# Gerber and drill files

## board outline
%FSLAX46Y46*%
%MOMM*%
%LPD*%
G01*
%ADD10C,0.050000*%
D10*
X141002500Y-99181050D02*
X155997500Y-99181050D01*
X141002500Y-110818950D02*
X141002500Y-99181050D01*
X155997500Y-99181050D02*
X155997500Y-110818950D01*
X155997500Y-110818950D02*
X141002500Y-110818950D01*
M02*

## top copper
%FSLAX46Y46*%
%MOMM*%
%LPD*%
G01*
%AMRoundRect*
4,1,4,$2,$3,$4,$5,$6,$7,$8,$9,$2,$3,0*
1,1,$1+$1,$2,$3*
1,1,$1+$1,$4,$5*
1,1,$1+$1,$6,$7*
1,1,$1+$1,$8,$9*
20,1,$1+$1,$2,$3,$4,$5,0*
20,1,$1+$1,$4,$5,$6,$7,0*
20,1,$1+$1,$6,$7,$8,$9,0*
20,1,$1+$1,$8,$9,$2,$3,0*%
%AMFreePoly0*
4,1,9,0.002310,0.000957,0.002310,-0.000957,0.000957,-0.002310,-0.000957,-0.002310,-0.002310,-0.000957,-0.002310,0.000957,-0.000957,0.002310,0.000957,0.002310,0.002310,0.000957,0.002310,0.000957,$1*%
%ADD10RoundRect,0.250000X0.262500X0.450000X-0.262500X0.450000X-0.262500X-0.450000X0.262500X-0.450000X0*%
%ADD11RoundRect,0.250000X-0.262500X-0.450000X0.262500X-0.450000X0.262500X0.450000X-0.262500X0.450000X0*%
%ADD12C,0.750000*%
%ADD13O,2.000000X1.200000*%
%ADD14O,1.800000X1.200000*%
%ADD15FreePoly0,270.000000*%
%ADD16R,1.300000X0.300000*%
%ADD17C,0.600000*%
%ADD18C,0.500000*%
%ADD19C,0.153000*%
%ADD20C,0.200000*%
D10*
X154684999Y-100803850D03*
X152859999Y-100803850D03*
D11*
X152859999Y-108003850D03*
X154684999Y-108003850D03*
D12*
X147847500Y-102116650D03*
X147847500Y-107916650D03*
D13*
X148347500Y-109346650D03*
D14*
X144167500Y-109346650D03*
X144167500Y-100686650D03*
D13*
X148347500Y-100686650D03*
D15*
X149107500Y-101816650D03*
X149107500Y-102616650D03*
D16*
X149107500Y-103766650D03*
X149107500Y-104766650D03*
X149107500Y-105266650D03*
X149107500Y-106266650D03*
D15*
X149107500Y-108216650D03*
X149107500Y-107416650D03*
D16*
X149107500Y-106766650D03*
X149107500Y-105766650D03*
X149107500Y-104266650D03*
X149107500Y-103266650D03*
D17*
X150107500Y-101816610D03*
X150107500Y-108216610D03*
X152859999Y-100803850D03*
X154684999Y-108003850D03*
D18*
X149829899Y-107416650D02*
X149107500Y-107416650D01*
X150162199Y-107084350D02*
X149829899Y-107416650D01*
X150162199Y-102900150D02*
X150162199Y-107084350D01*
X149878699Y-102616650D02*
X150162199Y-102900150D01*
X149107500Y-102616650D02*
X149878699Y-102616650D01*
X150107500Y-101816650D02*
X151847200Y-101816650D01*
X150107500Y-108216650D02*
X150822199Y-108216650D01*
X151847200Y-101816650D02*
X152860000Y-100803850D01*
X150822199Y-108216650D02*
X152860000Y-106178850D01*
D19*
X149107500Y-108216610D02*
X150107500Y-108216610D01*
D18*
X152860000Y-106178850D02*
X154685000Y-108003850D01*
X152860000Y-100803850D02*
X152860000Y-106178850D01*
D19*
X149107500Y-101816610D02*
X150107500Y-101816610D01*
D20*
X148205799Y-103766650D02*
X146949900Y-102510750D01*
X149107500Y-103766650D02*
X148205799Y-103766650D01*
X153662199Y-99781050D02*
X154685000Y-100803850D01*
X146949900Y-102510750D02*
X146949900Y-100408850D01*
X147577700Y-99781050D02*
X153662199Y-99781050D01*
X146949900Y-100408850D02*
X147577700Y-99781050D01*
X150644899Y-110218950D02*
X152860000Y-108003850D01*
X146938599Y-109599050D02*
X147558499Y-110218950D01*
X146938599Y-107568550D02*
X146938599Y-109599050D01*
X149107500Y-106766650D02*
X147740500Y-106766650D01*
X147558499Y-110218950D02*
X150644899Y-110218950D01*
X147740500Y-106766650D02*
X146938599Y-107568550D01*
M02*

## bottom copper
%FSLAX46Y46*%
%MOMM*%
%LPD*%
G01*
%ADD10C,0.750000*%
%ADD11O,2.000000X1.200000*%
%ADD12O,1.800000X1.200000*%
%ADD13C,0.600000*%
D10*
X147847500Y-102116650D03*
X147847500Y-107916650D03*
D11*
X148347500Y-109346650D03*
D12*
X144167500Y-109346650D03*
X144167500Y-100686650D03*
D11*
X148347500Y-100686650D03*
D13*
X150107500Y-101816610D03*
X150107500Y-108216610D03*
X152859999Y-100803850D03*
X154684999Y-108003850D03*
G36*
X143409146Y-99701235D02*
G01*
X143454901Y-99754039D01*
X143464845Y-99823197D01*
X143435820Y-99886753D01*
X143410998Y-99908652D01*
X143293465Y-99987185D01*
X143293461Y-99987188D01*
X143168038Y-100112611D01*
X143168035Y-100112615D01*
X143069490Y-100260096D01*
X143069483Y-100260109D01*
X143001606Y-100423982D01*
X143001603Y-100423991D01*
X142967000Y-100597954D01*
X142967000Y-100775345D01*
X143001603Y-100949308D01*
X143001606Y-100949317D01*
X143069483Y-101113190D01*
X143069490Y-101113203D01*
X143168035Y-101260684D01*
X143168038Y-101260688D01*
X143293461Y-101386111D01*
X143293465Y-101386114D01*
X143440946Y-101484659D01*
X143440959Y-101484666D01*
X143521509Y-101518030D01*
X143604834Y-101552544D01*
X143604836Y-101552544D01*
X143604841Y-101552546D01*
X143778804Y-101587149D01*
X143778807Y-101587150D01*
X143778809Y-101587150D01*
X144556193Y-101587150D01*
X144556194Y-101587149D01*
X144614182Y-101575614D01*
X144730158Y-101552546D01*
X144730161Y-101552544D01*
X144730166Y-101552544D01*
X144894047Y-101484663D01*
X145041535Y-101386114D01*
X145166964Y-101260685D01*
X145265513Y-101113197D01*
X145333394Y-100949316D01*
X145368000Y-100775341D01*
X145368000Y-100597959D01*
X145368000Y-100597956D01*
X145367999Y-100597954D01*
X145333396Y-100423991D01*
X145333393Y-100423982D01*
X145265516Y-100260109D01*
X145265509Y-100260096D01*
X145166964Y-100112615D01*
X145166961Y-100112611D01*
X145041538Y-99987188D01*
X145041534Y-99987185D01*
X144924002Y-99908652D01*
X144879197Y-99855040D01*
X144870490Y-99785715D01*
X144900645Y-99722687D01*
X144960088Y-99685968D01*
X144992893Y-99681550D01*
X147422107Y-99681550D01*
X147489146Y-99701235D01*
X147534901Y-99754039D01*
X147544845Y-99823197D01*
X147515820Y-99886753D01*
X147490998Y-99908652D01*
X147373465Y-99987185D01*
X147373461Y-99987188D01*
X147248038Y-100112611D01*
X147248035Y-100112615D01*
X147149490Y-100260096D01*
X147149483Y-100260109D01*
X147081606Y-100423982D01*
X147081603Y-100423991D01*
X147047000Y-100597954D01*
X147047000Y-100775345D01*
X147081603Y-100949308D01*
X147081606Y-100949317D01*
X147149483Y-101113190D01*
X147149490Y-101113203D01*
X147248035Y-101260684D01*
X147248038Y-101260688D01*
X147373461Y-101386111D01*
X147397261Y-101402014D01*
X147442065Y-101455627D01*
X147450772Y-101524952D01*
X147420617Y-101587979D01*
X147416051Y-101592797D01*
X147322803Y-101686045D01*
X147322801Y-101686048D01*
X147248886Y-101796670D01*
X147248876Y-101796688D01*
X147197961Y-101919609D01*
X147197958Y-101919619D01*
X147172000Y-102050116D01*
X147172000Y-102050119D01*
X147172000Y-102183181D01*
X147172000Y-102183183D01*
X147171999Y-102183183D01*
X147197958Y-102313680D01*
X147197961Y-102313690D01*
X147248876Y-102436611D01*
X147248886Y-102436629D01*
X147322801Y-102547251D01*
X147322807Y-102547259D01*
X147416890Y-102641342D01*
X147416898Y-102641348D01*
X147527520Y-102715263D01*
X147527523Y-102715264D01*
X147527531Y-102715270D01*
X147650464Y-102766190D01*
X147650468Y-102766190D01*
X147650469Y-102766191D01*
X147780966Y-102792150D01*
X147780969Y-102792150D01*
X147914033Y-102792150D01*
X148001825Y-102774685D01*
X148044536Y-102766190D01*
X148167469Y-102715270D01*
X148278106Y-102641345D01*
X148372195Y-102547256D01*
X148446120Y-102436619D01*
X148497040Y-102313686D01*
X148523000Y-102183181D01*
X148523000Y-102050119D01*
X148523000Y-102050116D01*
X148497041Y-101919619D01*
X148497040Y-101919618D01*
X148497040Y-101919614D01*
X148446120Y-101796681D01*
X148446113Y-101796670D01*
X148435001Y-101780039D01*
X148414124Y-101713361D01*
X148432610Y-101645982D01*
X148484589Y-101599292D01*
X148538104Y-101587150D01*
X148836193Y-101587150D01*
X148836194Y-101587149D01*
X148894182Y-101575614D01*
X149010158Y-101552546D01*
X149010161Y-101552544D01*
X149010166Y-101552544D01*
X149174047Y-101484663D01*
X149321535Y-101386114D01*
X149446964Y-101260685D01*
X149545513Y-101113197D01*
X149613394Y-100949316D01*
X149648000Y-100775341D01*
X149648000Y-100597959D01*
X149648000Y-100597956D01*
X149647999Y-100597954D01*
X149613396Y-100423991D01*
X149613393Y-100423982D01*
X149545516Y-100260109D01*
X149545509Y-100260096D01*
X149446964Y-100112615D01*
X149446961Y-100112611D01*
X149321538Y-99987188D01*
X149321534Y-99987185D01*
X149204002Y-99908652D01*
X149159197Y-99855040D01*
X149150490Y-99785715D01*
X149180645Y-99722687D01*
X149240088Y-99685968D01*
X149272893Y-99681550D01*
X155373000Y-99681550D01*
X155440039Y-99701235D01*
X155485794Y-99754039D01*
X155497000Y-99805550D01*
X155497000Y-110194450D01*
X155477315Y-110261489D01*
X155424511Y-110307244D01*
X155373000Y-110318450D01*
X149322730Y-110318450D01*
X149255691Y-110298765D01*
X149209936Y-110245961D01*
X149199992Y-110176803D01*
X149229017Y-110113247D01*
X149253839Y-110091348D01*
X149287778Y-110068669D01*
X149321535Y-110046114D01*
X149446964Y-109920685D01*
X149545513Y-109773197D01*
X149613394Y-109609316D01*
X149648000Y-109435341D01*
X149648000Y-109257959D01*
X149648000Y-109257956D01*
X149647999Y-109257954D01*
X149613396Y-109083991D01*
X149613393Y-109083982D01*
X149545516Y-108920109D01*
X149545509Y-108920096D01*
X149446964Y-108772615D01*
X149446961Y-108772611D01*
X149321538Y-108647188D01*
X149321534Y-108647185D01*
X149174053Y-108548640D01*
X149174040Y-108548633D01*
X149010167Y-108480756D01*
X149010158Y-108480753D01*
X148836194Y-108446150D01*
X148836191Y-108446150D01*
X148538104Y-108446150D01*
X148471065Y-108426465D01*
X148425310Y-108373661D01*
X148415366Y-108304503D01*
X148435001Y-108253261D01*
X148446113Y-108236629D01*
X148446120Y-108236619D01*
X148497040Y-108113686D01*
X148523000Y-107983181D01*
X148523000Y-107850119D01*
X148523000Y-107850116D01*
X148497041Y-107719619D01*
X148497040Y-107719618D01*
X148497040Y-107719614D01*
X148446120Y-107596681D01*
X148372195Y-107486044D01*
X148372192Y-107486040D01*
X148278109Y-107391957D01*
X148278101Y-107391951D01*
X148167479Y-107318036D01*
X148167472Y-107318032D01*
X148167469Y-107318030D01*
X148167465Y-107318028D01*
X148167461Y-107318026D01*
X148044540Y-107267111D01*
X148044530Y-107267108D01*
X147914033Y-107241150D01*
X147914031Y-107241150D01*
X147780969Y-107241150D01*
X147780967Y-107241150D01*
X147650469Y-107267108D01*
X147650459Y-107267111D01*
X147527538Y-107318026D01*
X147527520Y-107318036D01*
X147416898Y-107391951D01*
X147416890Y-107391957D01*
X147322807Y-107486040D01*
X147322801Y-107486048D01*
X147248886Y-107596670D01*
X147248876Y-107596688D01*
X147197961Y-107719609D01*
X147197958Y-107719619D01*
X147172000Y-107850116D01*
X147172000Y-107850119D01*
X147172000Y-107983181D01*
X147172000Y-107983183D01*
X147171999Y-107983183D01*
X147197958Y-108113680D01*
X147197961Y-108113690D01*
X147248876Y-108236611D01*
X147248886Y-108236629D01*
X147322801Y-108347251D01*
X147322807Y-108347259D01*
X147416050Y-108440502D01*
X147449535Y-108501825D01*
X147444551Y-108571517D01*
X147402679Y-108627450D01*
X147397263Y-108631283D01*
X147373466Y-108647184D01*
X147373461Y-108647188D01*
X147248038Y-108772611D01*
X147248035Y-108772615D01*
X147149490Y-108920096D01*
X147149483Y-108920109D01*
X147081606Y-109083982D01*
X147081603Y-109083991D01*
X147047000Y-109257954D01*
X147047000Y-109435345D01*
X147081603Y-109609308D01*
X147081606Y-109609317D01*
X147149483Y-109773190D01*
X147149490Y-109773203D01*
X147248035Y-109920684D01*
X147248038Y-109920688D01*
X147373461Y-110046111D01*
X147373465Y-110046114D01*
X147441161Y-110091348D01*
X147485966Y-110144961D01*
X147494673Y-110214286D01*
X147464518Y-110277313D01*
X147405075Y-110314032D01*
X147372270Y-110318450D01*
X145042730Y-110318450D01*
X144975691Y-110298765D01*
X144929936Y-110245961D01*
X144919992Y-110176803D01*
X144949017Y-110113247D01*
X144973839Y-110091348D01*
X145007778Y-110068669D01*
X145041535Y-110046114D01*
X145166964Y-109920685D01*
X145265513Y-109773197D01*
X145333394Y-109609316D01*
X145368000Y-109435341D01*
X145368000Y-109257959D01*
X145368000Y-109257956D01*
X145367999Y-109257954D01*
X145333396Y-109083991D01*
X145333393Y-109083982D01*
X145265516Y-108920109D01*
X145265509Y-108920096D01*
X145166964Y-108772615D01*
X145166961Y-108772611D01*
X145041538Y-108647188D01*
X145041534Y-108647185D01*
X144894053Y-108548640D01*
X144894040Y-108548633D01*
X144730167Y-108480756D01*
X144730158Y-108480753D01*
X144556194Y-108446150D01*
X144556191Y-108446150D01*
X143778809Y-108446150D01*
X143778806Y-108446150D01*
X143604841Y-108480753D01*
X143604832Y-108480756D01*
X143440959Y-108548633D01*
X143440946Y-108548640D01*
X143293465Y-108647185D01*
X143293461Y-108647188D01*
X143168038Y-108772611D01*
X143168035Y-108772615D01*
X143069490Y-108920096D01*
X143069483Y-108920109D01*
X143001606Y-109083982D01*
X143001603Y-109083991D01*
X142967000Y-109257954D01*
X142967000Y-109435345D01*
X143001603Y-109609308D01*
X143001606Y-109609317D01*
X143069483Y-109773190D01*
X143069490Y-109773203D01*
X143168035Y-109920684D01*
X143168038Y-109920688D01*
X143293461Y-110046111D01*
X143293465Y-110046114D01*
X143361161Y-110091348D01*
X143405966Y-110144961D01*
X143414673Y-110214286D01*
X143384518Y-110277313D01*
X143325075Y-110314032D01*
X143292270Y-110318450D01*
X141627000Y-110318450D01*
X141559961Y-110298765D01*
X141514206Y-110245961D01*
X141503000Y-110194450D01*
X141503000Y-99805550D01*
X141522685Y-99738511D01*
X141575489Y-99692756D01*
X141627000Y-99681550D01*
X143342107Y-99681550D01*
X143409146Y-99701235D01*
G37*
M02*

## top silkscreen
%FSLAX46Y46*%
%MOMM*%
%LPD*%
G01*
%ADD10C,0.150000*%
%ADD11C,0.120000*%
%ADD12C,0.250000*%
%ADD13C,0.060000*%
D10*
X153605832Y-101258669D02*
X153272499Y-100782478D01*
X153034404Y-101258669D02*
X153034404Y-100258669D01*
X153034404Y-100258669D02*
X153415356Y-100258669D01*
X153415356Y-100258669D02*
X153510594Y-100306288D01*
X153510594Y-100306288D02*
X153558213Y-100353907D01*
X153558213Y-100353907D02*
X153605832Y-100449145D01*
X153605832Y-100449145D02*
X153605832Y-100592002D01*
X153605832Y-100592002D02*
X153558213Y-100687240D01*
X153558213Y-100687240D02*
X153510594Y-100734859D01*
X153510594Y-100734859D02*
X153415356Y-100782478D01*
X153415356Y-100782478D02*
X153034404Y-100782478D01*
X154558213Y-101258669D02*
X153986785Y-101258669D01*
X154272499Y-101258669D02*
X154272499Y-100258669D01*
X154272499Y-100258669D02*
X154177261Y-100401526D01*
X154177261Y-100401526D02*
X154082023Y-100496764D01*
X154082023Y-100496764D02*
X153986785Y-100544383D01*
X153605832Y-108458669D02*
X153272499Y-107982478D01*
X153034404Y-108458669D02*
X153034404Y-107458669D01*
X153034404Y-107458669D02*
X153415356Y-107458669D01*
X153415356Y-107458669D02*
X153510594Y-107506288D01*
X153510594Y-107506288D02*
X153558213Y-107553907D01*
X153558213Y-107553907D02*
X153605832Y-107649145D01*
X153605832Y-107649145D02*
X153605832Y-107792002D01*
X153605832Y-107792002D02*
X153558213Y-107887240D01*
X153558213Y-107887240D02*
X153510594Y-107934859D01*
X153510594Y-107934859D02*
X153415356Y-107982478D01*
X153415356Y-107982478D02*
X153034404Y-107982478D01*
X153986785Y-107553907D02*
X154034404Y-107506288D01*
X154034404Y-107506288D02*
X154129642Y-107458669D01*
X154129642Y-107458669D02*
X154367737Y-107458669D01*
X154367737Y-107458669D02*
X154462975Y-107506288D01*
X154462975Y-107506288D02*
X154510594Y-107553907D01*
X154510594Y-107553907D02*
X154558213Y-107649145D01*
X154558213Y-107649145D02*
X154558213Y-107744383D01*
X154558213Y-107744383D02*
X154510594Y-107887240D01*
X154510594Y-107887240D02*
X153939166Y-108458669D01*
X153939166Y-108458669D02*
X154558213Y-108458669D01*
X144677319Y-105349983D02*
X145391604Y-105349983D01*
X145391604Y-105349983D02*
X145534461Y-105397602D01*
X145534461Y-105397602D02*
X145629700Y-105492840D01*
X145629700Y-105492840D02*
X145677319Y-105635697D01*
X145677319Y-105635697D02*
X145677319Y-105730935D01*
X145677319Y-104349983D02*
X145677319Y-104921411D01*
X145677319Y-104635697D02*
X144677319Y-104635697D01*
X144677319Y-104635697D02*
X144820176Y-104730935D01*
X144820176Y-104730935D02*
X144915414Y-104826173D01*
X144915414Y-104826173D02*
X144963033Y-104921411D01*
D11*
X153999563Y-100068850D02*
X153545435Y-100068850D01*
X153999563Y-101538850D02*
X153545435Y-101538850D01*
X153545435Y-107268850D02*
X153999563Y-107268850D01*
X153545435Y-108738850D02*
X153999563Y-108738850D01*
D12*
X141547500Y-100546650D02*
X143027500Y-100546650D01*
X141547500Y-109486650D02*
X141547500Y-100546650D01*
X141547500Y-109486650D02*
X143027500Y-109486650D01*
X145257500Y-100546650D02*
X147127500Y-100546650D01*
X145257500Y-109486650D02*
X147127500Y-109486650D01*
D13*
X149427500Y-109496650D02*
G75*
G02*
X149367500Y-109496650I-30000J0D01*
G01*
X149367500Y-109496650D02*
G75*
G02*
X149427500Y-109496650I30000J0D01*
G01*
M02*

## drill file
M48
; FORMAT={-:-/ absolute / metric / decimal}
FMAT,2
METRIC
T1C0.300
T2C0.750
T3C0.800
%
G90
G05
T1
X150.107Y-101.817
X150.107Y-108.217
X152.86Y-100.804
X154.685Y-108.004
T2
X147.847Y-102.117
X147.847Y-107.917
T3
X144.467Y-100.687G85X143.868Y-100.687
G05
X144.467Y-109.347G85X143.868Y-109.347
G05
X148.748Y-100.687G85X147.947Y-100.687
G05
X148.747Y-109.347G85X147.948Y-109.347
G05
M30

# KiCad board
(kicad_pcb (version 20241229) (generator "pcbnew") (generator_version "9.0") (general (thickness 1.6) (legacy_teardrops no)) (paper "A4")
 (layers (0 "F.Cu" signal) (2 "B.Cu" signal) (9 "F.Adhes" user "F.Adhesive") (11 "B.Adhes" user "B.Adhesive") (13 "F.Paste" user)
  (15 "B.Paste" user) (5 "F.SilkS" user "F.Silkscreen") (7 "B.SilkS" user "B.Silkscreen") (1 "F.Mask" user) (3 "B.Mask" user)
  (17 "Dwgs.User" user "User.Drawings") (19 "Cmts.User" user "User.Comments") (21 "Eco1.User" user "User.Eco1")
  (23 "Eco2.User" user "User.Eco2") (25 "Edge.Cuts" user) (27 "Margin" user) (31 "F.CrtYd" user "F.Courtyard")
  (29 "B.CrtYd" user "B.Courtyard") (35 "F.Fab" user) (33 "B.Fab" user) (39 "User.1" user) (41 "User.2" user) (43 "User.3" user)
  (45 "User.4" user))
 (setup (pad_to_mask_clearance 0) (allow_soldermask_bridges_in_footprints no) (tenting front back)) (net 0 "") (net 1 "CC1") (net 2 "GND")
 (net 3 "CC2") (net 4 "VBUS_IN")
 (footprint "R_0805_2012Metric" (layer "F.Cu") (at 153.772499 100.80385 180)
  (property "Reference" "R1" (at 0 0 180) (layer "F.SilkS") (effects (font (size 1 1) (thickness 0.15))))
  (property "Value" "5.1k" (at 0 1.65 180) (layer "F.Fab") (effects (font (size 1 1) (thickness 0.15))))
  (fp_line (start -0.227064 0.735) (end 0.227064 0.735) (stroke (width 0.12) (type solid)) (layer "F.SilkS"))
  (fp_line (start -0.227064 -0.735) (end 0.227064 -0.735) (stroke (width 0.12) (type solid)) (layer "F.SilkS"))
  (pad "1" smd roundrect (at -0.9125 0 180) (size 1.025 1.4) (layers "F.Cu" "F.Mask" "F.Paste") (roundrect_rratio 0.243902) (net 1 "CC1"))
  (pad "2" smd roundrect (at 0.9125 0 180) (size 1.025 1.4) (layers "F.Cu" "F.Mask" "F.Paste") (roundrect_rratio 0.243902) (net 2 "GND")))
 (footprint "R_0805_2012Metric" (layer "F.Cu") (at 153.772499 108.00385)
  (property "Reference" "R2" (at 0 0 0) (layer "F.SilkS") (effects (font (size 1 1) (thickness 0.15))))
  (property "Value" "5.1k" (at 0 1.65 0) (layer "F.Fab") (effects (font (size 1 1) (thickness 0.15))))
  (fp_line (start -0.227064 -0.735) (end 0.227064 -0.735) (stroke (width 0.12) (type solid)) (layer "F.SilkS"))
  (fp_line (start -0.227064 0.735) (end 0.227064 0.735) (stroke (width 0.12) (type solid)) (layer "F.SilkS"))
  (pad "1" smd roundrect (at -0.9125 0) (size 1.025 1.4) (layers "F.Cu" "F.Mask" "F.Paste") (roundrect_rratio 0.243902) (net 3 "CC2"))
  (pad "2" smd roundrect (at 0.9125 0) (size 1.025 1.4) (layers "F.Cu" "F.Mask" "F.Paste") (roundrect_rratio 0.243902) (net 2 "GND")))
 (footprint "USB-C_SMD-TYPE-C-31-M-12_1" (layer "F.Cu") (at 146.6375 105.01665 -90)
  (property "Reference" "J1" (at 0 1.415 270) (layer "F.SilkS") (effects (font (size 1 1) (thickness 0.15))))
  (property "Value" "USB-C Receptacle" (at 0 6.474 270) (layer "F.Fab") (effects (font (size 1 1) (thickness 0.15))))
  (fp_line (start -4.47 5.09) (end -4.47 3.61) (stroke (width 0.25) (type solid)) (layer "F.SilkS"))
  (fp_line (start 4.47 5.09) (end -4.47 5.09) (stroke (width 0.25) (type solid)) (layer "F.SilkS"))
  (fp_line (start 4.47 5.09) (end 4.47 3.61) (stroke (width 0.25) (type solid)) (layer "F.SilkS"))
  (fp_line (start -4.47 1.38) (end -4.47 -0.49) (stroke (width 0.25) (type solid)) (layer "F.SilkS"))
  (fp_line (start 4.47 1.38) (end 4.47 -0.49) (stroke (width 0.25) (type solid)) (layer "F.SilkS"))
  (fp_circle (center 4.48 -2.76) (end 4.51 -2.76) (stroke (width 0.06) (type solid)) (fill no) (layer "F.SilkS"))
  (pad "" thru_hole circle (at -2.9 -1.21 270) (size 0.75 0.75) (drill 0.75) (layers "*.Cu" "*.Mask") (remove_unused_layers no))
  (pad "" thru_hole circle (at 2.9 -1.21 270) (size 0.75 0.75) (drill 0.75) (layers "*.Cu" "*.Mask") (remove_unused_layers no))
  (pad "1" thru_hole oval (at 4.33 -1.71 270) (size 1.2 2) (drill oval 0.799998 1.599971) (layers "*.Cu" "*.Mask") (remove_unused_layers no))
  (pad "2" thru_hole oval (at 4.33 2.47 270) (size 1.2 1.8) (drill oval 0.799998 1.399997) (layers "*.Cu" "*.Mask")
   (remove_unused_layers no))
  (pad "3" thru_hole oval (at -4.33 2.47 270) (size 1.2 1.8) (drill oval 0.799998 1.399997) (layers "*.Cu" "*.Mask")
   (remove_unused_layers no))
  (pad "4" thru_hole oval (at -4.33 -1.71 270) (size 1.2 2) (drill oval 0.799998 1.600022) (layers "*.Cu" "*.Mask")
   (remove_unused_layers no))
  (pad "A1B12" smd custom (at -3.2 -2.47 270) (size 0.005 0.005) (layers "F.Cu" "F.Mask" "F.Paste") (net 2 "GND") (thermal_bridge_angle 90)
   (options (clearance outline) (anchor circle)) (primitives))
  (pad "A4B9" smd custom (at -2.4 -2.47 270) (size 0.005 0.005) (layers "F.Cu" "F.Mask" "F.Paste") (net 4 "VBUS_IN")
   (thermal_bridge_angle 90) (options (clearance outline) (anchor circle)) (primitives))
  (pad "A5" smd rect (at -1.25 -2.47 270) (size 0.3 1.3) (layers "F.Cu" "F.Mask" "F.Paste") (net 1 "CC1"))
  (pad "A6" smd rect (at -0.25 -2.47 270) (size 0.3 1.3) (layers "F.Cu" "F.Mask" "F.Paste"))
  (pad "A7" smd rect (at 0.25 -2.47 270) (size 0.3 1.3) (layers "F.Cu" "F.Mask" "F.Paste"))
  (pad "A8" smd rect (at 1.25 -2.47 270) (size 0.3 1.3) (layers "F.Cu" "F.Mask" "F.Paste"))
  (pad "B1A12" smd custom (at 3.2 -2.47 270) (size 0.005 0.005) (layers "F.Cu" "F.Mask" "F.Paste") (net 2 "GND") (thermal_bridge_angle 90)
   (options (clearance outline) (anchor circle)) (primitives))
  (pad "B4A9" smd custom (at 2.4 -2.47 270) (size 0.005 0.005) (layers "F.Cu" "F.Mask" "F.Paste") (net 4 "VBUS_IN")
   (thermal_bridge_angle 90) (options (clearance outline) (anchor circle)) (primitives))
  (pad "B5" smd rect (at 1.75 -2.47 270) (size 0.3 1.3) (layers "F.Cu" "F.Mask" "F.Paste") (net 3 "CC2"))
  (pad "B6" smd rect (at 0.75 -2.47 270) (size 0.3 1.3) (layers "F.Cu" "F.Mask" "F.Paste"))
  (pad "B7" smd rect (at -0.75 -2.47 270) (size 0.3 1.3) (layers "F.Cu" "F.Mask" "F.Paste"))
  (pad "B8" smd rect (at -1.75 -2.47 270) (size 0.3 1.3) (layers "F.Cu" "F.Mask" "F.Paste")))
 (gr_line (start 141.0025 99.18105) (end 155.9975 99.18105) (stroke (width 0.05) (type default)) (layer "Edge.Cuts"))
 (gr_line (start 141.0025 110.81895) (end 141.0025 99.18105) (stroke (width 0.05) (type default)) (layer "Edge.Cuts"))
 (gr_line (start 155.9975 99.18105) (end 155.9975 110.81895) (stroke (width 0.05) (type default)) (layer "Edge.Cuts"))
 (gr_line (start 155.9975 110.81895) (end 141.0025 110.81895) (stroke (width 0.05) (type default)) (layer "Edge.Cuts"))
 (segment (start 149.829899 107.41665) (end 149.1075 107.41665) (width 0.5) (layer "F.Cu") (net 4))
 (segment (start 150.162199 107.08435) (end 149.829899 107.41665) (width 0.5) (layer "F.Cu") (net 4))
 (segment (start 150.162199 102.90015) (end 150.162199 107.08435) (width 0.5) (layer "F.Cu") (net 4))
 (segment (start 149.878699 102.61665) (end 150.162199 102.90015) (width 0.5) (layer "F.Cu") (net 4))
 (segment (start 149.1075 102.61665) (end 149.878699 102.61665) (width 0.5) (layer "F.Cu") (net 4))
 (segment (start 150.1075 101.81665) (end 151.8472 101.81665) (width 0.5) (layer "F.Cu") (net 2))
 (segment (start 150.1075 108.21665) (end 150.822199 108.21665) (width 0.5) (layer "F.Cu") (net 2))
 (segment (start 151.8472 101.81665) (end 152.86 100.80385) (width 0.5) (layer "F.Cu") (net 2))
 (segment (start 150.822199 108.21665) (end 152.86 106.17885) (width 0.5) (layer "F.Cu") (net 2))
 (segment (start 149.1075 108.21661) (end 150.1075 108.21661) (width 0.153) (layer "F.Cu") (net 2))
 (segment (start 152.86 106.17885) (end 154.685 108.00385) (width 0.5) (layer "F.Cu") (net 2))
 (segment (start 152.86 100.80385) (end 152.86 106.17885) (width 0.5) (layer "F.Cu") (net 2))
 (segment (start 149.1075 101.81661) (end 150.1075 101.81661) (width 0.153) (layer "F.Cu") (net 2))
 (via (at 150.1075 101.81661) (size 0.6) (drill 0.3) (layers "F.Cu" "B.Cu") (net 2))
 (via (at 150.1075 108.21661) (size 0.6) (drill 0.3) (layers "F.Cu" "B.Cu") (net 2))
 (via (at 152.859999 100.80385) (size 0.6) (drill 0.3) (layers "F.Cu" "B.Cu") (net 2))
 (via (at 154.684999 108.00385) (size 0.6) (drill 0.3) (layers "F.Cu" "B.Cu") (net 2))
 (segment (start 148.205799 103.76665) (end 146.9499 102.51075) (width 0.2) (layer "F.Cu") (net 1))
 (segment (start 149.1075 103.76665) (end 148.205799 103.76665) (width 0.2) (layer "F.Cu") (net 1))
 (segment (start 153.662199 99.78105) (end 154.685 100.80385) (width 0.2) (layer "F.Cu") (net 1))
 (segment (start 146.9499 102.51075) (end 146.9499 100.40885) (width 0.2) (layer "F.Cu") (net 1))
 (segment (start 147.5777 99.78105) (end 153.662199 99.78105) (width 0.2) (layer "F.Cu") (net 1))
 (segment (start 146.9499 100.40885) (end 147.5777 99.78105) (width 0.2) (layer "F.Cu") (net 1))
 (segment (start 150.644899 110.21895) (end 152.86 108.00385) (width 0.2) (layer "F.Cu") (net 3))
 (segment (start 146.938599 109.59905) (end 147.558499 110.21895) (width 0.2) (layer "F.Cu") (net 3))
 (segment (start 146.938599 107.56855) (end 146.938599 109.59905) (width 0.2) (layer "F.Cu") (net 3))
 (segment (start 149.1075 106.76665) (end 147.7405 106.76665) (width 0.2) (layer "F.Cu") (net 3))
 (segment (start 147.558499 110.21895) (end 150.644899 110.21895) (width 0.2) (layer "F.Cu") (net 3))
 (segment (start 147.7405 106.76665) (end 146.938599 107.56855) (width 0.2) (layer "F.Cu") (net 3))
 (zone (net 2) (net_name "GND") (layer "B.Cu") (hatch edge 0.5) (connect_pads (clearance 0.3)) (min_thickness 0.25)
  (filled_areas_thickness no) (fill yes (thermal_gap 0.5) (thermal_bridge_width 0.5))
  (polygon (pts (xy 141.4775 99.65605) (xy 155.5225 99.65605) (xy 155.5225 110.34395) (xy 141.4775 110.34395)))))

